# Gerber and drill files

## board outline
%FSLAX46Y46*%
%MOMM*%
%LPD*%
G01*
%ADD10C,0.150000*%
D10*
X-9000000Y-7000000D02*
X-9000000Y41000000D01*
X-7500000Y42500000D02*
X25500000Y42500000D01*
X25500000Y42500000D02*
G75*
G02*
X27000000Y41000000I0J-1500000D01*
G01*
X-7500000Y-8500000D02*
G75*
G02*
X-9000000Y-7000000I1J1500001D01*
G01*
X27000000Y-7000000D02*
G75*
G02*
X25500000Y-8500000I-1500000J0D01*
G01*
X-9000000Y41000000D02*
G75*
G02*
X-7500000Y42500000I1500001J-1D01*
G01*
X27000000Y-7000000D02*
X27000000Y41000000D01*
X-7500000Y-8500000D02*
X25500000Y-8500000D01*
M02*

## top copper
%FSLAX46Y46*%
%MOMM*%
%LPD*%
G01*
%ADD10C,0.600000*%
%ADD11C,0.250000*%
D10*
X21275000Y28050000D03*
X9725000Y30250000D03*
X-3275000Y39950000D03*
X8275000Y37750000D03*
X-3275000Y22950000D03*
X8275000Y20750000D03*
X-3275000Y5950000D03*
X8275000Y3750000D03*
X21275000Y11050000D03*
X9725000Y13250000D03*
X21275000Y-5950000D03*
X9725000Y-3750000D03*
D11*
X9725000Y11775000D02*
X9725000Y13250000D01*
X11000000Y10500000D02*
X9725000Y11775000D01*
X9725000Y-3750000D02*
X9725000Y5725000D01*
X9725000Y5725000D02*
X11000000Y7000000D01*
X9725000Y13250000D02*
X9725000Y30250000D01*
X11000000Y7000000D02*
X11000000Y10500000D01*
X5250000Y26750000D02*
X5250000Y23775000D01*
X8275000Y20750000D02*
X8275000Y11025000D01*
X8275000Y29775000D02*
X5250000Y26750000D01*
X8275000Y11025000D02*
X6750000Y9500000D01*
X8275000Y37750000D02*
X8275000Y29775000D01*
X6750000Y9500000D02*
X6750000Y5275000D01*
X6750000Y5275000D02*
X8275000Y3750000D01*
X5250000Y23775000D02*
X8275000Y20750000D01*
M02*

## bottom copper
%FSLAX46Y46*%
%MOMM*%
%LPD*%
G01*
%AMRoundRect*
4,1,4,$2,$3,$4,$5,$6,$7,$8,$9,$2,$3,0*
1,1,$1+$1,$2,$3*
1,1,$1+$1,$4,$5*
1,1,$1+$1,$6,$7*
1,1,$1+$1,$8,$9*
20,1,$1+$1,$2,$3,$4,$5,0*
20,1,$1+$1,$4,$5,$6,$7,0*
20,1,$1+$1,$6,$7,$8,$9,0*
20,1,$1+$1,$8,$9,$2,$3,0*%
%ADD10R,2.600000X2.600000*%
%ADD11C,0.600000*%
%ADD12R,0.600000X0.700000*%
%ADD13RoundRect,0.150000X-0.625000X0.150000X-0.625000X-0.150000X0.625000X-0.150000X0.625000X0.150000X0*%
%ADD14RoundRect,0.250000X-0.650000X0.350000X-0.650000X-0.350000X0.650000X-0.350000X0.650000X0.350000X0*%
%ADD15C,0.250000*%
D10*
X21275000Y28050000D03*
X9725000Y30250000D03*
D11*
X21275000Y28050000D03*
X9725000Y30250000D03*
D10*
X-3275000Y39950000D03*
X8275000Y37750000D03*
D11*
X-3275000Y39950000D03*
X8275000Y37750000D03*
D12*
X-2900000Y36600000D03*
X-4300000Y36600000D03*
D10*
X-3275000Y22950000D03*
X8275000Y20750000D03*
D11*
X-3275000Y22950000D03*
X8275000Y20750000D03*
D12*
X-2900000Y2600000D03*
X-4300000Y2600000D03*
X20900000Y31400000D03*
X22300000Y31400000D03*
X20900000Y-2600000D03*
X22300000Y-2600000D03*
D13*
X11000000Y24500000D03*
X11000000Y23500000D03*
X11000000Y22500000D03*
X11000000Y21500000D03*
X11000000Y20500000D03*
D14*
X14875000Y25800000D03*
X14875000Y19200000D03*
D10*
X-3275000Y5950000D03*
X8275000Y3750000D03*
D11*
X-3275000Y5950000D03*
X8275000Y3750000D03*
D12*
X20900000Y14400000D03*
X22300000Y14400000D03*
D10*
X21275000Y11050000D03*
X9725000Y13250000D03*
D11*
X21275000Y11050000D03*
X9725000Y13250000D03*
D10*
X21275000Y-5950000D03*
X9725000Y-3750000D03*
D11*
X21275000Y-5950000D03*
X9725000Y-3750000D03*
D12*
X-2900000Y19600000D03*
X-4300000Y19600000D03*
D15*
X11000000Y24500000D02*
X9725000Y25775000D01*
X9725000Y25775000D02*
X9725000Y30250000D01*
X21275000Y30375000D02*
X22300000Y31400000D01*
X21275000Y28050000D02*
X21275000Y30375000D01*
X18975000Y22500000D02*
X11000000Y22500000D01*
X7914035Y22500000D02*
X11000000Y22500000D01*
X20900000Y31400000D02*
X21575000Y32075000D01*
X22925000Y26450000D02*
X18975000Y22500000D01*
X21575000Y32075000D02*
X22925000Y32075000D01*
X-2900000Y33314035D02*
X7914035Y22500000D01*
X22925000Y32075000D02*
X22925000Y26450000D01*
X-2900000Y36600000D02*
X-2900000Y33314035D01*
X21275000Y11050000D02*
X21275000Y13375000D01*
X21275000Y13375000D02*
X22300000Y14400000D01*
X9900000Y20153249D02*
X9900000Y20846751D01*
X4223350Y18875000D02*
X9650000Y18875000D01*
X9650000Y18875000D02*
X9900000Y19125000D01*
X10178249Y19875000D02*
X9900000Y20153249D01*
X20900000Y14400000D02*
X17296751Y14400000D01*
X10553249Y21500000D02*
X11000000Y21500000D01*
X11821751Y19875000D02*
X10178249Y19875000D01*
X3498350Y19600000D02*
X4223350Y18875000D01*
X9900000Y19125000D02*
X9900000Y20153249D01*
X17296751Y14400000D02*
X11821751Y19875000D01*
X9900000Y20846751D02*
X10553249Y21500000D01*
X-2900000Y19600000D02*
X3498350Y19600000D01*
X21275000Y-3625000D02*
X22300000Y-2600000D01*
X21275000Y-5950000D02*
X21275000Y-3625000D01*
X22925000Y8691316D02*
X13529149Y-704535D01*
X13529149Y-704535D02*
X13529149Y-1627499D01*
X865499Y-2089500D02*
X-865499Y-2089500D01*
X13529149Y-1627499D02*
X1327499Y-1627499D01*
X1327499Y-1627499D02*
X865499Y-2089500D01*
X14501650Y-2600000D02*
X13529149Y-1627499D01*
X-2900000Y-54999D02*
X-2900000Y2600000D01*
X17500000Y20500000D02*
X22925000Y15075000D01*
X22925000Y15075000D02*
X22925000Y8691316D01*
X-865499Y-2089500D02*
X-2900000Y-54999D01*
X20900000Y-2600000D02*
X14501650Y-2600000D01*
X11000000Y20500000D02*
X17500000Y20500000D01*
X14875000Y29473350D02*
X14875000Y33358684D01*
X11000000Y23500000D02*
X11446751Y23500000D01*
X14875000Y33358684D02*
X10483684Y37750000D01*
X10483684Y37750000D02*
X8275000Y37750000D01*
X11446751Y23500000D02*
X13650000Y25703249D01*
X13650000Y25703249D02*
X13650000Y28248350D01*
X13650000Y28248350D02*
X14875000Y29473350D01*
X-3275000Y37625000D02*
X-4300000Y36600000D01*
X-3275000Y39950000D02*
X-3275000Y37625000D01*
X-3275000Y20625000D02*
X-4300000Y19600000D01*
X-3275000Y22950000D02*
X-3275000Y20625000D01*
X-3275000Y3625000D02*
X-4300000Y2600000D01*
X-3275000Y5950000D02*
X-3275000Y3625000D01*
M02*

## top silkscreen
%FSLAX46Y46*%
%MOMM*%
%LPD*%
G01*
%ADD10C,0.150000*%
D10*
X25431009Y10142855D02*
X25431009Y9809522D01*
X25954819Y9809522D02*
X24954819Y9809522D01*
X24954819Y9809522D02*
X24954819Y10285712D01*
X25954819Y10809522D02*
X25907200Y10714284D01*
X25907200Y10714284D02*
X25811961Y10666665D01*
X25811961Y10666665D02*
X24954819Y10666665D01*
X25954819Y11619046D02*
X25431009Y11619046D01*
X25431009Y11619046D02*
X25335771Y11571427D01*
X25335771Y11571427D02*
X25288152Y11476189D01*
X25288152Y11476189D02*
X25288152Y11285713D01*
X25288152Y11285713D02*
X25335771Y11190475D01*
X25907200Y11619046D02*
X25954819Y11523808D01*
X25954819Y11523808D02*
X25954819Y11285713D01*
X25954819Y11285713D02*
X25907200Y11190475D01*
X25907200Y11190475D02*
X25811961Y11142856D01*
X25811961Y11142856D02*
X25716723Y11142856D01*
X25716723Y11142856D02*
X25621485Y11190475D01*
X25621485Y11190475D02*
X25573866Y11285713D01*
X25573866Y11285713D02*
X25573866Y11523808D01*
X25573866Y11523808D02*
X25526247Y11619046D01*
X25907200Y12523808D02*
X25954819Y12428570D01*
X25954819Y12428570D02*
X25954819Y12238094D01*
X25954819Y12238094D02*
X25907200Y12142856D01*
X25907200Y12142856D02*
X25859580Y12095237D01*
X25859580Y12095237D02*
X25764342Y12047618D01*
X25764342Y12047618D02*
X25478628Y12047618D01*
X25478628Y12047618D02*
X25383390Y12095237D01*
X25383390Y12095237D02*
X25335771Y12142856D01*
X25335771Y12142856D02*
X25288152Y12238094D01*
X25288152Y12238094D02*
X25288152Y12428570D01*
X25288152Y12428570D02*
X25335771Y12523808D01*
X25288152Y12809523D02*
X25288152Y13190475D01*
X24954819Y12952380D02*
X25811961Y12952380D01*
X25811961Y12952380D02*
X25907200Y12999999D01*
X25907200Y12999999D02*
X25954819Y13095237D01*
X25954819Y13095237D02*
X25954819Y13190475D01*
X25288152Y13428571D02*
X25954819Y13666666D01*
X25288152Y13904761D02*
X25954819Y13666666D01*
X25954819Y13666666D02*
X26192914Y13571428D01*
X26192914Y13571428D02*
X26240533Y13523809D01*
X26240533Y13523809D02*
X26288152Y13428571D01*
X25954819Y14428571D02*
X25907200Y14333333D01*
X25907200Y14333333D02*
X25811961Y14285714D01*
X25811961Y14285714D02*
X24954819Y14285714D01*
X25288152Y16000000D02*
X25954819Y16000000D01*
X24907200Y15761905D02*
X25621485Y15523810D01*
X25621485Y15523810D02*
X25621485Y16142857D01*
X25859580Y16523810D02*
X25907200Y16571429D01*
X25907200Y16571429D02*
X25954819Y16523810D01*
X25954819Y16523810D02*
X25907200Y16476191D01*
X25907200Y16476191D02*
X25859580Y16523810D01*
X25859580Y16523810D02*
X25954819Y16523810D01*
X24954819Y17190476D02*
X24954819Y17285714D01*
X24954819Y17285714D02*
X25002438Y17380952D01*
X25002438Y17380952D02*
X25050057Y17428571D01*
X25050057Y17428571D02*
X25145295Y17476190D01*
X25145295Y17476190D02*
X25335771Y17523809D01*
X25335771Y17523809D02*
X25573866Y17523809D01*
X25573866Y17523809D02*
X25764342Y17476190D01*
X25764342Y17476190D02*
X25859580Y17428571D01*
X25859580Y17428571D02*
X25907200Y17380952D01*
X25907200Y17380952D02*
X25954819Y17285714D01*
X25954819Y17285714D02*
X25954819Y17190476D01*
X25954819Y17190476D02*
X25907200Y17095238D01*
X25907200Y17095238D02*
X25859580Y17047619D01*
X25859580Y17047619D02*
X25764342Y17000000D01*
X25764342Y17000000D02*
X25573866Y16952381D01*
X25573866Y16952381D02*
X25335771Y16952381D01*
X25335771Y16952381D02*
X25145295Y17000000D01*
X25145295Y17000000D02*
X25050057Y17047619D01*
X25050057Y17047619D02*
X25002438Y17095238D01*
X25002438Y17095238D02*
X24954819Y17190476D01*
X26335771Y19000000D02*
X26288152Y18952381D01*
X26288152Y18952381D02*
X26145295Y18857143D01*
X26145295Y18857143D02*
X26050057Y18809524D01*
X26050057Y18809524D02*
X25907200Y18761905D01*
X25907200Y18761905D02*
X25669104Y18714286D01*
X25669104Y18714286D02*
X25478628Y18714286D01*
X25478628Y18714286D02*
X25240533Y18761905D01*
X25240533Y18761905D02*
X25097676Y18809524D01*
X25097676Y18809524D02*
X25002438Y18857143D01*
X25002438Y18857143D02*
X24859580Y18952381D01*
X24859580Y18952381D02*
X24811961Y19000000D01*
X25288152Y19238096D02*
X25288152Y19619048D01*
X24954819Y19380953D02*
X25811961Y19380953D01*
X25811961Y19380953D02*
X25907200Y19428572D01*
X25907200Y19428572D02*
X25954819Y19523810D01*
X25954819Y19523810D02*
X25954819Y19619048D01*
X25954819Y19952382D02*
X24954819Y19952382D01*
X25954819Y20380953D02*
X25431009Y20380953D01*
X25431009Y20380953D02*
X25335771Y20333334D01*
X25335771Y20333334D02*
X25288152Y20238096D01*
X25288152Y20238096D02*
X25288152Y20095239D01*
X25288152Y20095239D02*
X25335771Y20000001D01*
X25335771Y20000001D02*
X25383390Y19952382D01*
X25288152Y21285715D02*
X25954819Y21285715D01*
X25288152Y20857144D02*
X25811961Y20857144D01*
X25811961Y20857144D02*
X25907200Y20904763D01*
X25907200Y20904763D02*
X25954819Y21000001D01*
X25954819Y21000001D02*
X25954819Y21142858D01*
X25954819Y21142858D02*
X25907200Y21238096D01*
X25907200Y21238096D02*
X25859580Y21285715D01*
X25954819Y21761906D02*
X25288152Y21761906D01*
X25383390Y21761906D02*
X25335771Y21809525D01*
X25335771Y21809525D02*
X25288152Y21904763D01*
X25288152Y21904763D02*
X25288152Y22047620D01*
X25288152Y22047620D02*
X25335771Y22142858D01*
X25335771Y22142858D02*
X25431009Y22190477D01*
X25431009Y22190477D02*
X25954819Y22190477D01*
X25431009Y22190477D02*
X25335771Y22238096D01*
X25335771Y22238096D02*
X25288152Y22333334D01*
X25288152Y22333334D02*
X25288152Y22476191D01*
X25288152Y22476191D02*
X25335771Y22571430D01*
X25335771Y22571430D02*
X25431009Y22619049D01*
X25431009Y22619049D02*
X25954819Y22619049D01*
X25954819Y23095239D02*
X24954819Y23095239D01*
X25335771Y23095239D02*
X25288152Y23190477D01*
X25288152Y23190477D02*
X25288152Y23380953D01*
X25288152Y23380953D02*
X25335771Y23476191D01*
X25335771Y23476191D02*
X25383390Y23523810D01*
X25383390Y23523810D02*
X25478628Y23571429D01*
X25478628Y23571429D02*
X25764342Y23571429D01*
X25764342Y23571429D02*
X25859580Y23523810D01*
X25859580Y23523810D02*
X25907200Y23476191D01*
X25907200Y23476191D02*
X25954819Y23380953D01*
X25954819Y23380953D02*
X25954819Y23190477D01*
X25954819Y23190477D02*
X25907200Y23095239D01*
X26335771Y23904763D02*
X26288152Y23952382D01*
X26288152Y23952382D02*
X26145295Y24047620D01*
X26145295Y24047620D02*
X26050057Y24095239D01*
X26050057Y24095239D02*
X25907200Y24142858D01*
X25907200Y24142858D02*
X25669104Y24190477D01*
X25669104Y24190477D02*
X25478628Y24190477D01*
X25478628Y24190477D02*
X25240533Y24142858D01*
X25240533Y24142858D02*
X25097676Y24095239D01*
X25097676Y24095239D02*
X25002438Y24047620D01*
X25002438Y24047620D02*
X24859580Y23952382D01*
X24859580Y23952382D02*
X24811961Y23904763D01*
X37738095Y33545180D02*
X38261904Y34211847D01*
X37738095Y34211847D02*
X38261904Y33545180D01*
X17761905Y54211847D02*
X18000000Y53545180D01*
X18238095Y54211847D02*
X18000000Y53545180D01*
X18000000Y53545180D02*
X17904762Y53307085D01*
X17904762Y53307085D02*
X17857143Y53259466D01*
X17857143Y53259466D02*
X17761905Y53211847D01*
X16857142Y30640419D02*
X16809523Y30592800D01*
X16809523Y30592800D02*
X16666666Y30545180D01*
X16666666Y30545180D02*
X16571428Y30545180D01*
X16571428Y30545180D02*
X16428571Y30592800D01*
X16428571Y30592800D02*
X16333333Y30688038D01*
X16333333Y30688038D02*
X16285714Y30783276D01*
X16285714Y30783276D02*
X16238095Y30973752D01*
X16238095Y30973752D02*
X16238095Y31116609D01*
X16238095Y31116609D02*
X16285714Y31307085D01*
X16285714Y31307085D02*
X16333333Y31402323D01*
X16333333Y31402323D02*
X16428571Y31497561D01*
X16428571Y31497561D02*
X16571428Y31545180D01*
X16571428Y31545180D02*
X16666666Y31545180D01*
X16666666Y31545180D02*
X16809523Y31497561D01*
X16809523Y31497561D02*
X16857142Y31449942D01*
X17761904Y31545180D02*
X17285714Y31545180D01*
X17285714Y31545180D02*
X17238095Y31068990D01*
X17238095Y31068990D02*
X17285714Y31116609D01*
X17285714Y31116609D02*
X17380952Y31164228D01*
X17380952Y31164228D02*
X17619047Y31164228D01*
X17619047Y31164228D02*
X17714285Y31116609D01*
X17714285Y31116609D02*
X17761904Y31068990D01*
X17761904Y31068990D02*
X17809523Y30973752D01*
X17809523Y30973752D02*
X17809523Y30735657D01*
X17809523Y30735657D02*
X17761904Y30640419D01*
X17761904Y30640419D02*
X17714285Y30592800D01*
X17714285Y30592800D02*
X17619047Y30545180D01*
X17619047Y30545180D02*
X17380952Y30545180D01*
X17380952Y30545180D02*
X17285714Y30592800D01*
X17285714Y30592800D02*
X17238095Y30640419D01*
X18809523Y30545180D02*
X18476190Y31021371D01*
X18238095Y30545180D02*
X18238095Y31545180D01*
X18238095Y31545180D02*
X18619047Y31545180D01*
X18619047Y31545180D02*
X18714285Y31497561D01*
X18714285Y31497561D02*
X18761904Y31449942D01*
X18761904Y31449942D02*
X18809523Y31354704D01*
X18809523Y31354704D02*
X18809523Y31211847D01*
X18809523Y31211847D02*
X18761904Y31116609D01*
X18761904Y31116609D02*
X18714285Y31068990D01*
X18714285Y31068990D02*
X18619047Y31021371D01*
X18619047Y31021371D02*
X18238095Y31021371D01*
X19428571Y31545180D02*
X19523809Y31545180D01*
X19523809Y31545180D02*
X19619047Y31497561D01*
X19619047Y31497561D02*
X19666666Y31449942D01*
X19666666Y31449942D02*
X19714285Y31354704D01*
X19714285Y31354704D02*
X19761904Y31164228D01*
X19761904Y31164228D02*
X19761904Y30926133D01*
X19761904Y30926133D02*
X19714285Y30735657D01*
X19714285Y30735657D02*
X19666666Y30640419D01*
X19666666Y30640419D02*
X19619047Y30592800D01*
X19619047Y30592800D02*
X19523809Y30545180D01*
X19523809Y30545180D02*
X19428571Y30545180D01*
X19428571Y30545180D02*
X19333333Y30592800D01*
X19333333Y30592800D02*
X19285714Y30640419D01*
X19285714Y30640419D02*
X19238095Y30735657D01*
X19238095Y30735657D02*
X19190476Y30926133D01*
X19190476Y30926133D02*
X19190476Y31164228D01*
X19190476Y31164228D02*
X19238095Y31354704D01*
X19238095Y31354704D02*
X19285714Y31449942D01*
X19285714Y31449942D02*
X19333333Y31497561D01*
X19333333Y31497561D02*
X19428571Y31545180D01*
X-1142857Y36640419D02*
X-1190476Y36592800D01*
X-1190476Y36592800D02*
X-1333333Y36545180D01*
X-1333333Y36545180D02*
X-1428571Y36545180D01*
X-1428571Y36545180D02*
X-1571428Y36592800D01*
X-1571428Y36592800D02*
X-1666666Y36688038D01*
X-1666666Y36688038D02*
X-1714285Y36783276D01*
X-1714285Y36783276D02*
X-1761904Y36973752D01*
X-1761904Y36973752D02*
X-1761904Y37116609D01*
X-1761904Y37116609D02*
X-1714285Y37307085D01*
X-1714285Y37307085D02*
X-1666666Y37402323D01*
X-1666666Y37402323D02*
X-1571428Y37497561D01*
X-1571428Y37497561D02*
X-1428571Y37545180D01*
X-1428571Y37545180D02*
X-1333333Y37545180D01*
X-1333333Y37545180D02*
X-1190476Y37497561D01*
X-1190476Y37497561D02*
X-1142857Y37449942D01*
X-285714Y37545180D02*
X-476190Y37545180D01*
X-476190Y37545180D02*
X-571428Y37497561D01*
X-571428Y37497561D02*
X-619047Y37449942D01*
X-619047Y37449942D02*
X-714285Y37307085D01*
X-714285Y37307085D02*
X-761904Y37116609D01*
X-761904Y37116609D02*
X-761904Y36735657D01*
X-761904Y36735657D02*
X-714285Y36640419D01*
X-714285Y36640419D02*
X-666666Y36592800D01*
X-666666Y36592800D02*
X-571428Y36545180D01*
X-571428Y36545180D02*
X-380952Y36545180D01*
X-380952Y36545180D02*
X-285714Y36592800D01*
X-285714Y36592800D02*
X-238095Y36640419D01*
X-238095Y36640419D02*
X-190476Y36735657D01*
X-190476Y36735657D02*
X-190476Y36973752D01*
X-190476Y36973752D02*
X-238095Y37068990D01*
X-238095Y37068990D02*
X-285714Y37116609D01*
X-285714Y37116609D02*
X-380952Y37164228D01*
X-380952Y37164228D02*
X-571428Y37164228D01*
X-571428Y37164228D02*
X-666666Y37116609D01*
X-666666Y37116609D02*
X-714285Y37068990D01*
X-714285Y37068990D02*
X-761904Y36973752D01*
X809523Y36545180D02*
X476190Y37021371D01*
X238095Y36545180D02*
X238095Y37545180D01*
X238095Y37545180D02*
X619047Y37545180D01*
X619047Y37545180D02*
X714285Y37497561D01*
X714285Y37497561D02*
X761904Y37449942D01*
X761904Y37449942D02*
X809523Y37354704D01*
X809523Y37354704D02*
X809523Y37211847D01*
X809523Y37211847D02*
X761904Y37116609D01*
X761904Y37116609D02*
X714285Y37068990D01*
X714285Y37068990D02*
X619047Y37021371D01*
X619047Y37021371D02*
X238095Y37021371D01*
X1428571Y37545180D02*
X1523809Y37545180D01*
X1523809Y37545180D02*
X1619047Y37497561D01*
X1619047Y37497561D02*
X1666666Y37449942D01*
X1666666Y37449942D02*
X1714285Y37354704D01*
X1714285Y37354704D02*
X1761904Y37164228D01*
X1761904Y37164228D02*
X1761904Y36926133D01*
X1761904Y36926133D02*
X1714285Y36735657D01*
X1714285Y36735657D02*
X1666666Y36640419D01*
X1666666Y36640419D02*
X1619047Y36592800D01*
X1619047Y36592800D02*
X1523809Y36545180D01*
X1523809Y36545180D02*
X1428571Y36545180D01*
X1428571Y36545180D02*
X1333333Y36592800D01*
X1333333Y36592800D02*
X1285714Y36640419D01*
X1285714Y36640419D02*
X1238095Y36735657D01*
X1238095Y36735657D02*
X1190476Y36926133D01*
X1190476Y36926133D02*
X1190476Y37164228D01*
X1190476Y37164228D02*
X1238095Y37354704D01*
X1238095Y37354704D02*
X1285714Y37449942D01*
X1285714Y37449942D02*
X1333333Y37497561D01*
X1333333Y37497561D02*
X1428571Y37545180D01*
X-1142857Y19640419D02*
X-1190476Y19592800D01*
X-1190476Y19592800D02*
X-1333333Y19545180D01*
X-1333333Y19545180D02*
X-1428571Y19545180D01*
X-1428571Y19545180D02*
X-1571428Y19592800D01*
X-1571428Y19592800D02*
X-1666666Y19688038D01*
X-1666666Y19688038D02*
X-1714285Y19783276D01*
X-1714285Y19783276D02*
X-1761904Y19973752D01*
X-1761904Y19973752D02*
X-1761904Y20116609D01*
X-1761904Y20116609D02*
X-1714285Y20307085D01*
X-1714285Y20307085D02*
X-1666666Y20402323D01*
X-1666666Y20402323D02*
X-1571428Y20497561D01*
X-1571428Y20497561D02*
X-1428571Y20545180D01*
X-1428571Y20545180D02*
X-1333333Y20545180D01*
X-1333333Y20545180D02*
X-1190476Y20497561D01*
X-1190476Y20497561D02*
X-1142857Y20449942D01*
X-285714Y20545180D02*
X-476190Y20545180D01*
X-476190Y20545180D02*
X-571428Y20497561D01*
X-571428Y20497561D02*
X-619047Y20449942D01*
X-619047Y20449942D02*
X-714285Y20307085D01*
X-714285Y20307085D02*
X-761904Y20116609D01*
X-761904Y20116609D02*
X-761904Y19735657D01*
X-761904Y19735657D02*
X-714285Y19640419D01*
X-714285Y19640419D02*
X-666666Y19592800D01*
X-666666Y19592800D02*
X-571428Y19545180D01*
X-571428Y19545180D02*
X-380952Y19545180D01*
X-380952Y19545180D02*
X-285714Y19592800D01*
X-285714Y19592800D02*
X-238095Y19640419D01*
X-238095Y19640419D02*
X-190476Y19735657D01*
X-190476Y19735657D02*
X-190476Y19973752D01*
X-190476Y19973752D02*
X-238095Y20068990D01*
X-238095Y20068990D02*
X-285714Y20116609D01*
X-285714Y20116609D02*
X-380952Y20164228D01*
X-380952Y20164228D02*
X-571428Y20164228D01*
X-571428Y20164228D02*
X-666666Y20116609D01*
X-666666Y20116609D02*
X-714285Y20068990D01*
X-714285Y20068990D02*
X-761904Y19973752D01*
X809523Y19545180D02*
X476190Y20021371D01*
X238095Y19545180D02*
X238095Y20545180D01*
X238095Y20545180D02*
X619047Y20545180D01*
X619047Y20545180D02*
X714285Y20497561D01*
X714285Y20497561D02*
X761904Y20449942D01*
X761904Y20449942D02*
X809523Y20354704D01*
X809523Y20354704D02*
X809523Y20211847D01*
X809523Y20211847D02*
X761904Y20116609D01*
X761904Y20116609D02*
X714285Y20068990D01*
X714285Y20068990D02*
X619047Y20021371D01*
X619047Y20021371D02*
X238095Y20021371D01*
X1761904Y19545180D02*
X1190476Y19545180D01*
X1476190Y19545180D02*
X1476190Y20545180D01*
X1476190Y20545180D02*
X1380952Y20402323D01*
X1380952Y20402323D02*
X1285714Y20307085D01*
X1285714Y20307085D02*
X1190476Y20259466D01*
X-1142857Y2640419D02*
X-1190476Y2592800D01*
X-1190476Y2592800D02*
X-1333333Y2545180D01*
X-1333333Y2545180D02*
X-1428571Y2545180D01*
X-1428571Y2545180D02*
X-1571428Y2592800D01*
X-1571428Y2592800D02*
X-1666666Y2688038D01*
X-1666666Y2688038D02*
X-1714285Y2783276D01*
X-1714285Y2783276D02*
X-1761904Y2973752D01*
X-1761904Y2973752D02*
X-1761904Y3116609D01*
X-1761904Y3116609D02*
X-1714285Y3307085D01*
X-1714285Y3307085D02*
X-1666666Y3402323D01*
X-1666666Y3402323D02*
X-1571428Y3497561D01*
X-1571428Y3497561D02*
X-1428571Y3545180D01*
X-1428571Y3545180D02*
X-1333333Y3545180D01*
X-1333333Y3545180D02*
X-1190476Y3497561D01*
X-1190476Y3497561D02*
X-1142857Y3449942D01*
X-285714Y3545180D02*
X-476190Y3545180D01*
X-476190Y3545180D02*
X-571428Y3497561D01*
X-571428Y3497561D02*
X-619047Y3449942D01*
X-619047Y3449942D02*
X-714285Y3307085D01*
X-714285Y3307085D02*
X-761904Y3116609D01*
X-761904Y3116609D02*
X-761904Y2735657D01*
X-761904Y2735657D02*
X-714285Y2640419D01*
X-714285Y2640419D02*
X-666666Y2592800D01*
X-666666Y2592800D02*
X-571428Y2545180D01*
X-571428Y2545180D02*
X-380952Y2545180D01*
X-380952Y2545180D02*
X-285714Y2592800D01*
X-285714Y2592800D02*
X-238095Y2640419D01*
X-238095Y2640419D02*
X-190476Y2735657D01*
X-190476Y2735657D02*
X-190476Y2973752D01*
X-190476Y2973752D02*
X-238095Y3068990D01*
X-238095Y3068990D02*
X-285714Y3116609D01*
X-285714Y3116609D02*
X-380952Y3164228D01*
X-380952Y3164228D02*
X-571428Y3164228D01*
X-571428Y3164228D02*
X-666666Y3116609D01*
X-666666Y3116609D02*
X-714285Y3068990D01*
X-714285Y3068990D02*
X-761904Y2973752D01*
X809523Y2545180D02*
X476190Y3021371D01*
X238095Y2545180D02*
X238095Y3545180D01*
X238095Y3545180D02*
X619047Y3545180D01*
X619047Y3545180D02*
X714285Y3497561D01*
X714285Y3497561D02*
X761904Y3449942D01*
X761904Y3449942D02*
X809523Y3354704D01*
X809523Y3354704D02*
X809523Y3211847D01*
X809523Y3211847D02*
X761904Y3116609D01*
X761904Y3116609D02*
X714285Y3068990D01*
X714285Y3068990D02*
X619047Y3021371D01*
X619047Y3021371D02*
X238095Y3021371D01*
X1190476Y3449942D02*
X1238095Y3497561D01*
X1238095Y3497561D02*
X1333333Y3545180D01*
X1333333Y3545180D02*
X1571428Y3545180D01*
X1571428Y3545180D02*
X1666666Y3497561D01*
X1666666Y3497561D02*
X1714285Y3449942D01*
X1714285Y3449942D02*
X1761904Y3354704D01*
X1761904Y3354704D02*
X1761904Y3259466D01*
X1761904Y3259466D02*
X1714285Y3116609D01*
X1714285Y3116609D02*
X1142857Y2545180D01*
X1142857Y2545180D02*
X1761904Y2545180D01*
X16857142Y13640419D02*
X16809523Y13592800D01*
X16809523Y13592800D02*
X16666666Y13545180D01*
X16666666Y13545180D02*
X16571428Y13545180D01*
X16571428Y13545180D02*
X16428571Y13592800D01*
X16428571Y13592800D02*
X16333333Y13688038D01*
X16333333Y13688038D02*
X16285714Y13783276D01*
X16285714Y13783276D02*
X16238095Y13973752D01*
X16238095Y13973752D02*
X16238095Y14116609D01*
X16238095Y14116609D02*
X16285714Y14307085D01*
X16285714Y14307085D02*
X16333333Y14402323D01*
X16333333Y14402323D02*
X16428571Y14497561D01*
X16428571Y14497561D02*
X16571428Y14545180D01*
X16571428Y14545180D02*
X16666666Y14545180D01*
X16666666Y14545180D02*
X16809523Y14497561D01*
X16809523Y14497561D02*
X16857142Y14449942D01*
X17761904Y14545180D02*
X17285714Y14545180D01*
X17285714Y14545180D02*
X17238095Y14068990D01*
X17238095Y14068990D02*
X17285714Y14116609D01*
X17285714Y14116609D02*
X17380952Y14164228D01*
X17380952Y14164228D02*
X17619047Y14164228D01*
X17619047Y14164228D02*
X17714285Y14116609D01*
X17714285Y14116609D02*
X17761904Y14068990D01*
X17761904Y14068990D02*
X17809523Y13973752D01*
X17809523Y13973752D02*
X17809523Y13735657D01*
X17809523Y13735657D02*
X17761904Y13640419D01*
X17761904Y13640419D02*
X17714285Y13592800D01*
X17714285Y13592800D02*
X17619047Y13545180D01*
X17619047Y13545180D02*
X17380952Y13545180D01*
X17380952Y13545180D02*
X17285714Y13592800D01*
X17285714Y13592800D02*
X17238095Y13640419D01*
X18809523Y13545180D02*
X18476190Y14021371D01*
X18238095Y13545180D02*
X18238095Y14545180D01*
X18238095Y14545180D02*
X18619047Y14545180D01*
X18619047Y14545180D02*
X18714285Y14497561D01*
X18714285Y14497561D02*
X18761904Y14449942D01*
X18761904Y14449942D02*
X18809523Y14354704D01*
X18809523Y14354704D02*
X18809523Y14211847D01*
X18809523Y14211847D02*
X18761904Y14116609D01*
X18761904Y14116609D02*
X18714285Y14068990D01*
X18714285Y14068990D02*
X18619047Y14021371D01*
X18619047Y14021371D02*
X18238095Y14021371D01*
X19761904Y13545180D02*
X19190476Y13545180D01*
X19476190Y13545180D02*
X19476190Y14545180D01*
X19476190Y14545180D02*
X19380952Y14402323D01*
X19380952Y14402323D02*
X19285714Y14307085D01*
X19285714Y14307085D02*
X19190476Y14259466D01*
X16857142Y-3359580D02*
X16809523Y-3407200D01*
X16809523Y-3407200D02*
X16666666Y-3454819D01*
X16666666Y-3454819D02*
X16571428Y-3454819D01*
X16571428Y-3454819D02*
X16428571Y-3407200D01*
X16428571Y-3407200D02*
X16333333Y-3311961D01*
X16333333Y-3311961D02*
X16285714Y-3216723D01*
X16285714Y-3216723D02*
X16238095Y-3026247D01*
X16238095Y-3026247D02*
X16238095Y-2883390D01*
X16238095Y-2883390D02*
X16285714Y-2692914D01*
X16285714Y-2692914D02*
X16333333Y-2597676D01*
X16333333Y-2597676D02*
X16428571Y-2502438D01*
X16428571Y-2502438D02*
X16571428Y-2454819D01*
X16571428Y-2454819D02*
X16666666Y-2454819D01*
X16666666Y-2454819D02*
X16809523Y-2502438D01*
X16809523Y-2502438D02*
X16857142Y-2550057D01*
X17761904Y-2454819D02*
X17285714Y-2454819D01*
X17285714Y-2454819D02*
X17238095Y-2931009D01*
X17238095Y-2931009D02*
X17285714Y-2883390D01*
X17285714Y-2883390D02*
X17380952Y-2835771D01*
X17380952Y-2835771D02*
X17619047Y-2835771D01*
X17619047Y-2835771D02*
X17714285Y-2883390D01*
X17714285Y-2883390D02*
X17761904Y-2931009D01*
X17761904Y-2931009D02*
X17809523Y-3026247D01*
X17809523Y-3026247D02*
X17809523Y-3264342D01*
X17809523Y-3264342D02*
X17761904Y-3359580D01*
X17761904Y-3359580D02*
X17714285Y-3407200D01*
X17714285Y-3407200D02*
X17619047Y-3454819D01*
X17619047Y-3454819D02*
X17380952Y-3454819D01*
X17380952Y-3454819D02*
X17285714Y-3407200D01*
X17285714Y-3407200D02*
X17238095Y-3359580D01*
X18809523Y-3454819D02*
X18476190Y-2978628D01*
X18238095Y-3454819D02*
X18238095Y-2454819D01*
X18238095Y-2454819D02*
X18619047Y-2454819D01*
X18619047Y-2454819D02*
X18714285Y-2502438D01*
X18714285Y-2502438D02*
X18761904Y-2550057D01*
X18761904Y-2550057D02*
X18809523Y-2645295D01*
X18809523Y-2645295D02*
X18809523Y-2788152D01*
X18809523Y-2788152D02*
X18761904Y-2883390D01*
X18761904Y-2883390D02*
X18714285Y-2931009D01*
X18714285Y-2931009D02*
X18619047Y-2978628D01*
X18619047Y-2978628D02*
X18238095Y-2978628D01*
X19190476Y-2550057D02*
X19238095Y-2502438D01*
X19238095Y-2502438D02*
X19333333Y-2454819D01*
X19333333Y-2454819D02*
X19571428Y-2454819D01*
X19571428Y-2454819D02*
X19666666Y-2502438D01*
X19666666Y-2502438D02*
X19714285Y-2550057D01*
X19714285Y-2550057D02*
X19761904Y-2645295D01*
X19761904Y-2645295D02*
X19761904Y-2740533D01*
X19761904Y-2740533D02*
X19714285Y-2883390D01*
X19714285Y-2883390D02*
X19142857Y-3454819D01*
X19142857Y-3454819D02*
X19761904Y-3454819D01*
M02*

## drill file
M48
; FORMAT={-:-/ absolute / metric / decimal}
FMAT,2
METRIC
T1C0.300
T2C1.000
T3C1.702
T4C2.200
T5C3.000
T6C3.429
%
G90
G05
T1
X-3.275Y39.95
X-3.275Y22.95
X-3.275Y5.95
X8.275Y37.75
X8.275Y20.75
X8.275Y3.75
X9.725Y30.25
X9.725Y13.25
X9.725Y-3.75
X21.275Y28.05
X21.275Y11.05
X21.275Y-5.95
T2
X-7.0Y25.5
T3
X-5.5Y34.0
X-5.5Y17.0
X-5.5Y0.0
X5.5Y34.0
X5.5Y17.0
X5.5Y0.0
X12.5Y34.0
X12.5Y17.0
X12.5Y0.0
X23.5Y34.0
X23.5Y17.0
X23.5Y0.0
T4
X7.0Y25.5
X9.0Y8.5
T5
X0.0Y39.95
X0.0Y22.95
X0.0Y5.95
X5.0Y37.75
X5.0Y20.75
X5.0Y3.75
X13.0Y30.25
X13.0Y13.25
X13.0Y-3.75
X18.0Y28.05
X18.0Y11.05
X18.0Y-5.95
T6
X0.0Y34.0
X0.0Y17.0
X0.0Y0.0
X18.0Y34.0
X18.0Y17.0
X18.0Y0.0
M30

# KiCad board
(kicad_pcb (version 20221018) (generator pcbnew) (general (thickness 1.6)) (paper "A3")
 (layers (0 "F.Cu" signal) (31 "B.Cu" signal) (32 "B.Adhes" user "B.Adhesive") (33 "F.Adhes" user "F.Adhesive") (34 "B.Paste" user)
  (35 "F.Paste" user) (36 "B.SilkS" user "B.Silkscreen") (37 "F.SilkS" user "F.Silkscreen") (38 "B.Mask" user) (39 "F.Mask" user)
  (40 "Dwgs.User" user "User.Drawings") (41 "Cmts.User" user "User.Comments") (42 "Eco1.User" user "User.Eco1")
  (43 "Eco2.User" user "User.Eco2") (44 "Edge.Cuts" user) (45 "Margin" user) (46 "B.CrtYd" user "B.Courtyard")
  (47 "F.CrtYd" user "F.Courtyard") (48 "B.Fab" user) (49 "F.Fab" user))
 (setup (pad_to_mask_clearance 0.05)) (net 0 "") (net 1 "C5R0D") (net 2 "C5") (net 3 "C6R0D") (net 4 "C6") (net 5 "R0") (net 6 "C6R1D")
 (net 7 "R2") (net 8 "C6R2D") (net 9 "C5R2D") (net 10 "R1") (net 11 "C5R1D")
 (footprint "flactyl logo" (layer "F.Cu") (at 25.5 -17 -90)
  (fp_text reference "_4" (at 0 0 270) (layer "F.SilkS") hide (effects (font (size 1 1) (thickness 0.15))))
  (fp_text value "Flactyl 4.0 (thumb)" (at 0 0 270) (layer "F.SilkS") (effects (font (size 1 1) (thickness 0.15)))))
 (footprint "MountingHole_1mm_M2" (layer "F.Cu") (at -7 -25.5)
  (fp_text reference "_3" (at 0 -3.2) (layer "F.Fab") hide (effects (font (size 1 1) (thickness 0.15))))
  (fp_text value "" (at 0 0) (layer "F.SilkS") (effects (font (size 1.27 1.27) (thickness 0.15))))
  (pad "" np_thru_hole circle (at 0 0) (size 1 1) (drill 1) (layers "*.Cu" "*.Mask")))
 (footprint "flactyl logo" (layer "F.Cu") (at 38 -34)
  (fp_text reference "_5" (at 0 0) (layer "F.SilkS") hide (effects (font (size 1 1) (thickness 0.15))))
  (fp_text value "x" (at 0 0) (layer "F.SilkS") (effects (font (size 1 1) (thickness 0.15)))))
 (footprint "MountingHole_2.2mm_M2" (layer "F.Cu") (at 7 -25.5)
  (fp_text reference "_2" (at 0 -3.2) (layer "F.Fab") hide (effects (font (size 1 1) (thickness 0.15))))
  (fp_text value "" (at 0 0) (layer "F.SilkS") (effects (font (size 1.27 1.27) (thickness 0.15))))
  (pad "" np_thru_hole circle (at 0 0) (size 2.2 2.2) (drill 2.2) (layers "*.Cu" "*.Mask")))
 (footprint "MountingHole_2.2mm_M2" (layer "F.Cu") (at 9 -8.5)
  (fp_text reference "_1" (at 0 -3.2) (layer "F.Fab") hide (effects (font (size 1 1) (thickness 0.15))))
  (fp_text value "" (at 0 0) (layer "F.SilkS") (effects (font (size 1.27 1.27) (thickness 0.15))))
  (pad "" np_thru_hole circle (at 0 0) (size 2.2 2.2) (drill 2.2) (layers "*.Cu" "*.Mask")))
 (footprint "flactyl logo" (layer "F.Cu") (at 18 -54)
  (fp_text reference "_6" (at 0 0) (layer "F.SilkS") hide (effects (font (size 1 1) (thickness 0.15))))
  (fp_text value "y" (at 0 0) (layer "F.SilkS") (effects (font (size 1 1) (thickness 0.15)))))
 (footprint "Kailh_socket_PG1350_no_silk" (layer "B.Cu") (at 18 -34)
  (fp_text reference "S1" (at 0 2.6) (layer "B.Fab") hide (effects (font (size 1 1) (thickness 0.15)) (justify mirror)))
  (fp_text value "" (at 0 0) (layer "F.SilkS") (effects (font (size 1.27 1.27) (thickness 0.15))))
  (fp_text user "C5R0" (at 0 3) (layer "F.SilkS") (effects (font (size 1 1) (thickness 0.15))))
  (pad "" np_thru_hole circle (at -5.5 0) (size 1.7018 1.7018) (drill 1.7018) (layers "*.Cu" "*.Mask"))
  (pad "" np_thru_hole circle (at -5 3.75) (size 3 3) (drill 3) (layers "*.Cu" "*.Mask"))
  (pad "" np_thru_hole circle (at 0 0) (size 3.429 3.429) (drill 3.429) (layers "*.Cu" "*.Mask"))
  (pad "" np_thru_hole circle (at 0 5.95) (size 3 3) (drill 3) (layers "*.Cu" "*.Mask"))
  (pad "" np_thru_hole circle (at 5.5 0) (size 1.7018 1.7018) (drill 1.7018) (layers "*.Cu" "*.Mask"))
  (pad "1" smd rect (at 3.275 5.95) (size 2.6 2.6) (layers "B.Cu" "B.Paste" "B.Mask") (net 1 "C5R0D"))
  (pad "2" smd rect (at -8.275 3.75) (size 2.6 2.6) (layers "B.Cu" "B.Paste" "B.Mask") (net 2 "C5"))
  (pad "3" thru_hole circle (at 3.275 5.95) (size 0.6 0.6) (drill 0.3) (layers "*.Cu") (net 1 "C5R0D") (zone_connect 2))
  (pad "4" thru_hole circle (at -8.275 3.75) (size 0.6 0.6) (drill 0.3) (layers "*.Cu") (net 2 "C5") (zone_connect 2)))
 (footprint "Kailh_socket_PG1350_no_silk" (layer "B.Cu") (at 0 -34 180)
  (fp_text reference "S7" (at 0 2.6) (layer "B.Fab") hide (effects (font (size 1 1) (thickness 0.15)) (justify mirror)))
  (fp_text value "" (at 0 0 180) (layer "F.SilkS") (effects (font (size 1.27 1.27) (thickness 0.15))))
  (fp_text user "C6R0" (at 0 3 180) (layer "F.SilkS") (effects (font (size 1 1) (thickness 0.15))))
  (pad "" np_thru_hole circle (at -5.5 0) (size 1.7018 1.7018) (drill 1.7018) (layers "*.Cu" "*.Mask"))
  (pad "" np_thru_hole circle (at -5 3.75) (size 3 3) (drill 3) (layers "*.Cu" "*.Mask"))
  (pad "" np_thru_hole circle (at 0 0) (size 3.429 3.429) (drill 3.429) (layers "*.Cu" "*.Mask"))
  (pad "" np_thru_hole circle (at 0 5.95) (size 3 3) (drill 3) (layers "*.Cu" "*.Mask"))
  (pad "" np_thru_hole circle (at 5.5 0) (size 1.7018 1.7018) (drill 1.7018) (layers "*.Cu" "*.Mask"))
  (pad "1" smd rect (at 3.275 5.95) (size 2.6 2.6) (layers "B.Cu" "B.Paste" "B.Mask") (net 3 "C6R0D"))
  (pad "2" smd rect (at -8.275 3.75) (size 2.6 2.6) (layers "B.Cu" "B.Paste" "B.Mask") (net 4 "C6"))
  (pad "3" thru_hole circle (at 3.275 5.95) (size 0.6 0.6) (drill 0.3) (layers "*.Cu") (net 3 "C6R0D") (zone_connect 2))
  (pad "4" thru_hole circle (at -8.275 3.75) (size 0.6 0.6) (drill 0.3) (layers "*.Cu") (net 4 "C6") (zone_connect 2)))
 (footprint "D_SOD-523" (layer "B.Cu") (at -3.6 -36.6 180)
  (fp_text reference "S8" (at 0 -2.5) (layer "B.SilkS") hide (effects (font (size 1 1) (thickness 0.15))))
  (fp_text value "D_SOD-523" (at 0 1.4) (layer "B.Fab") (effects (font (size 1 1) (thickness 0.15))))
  (pad "1" smd rect (at -0.7 0 180) (size 0.6 0.7) (layers "B.Cu" "B.Paste" "B.Mask") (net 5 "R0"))
  (pad "2" smd rect (at 0.7 0 180) (size 0.6 0.7) (layers "B.Cu" "B.Paste" "B.Mask") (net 3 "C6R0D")))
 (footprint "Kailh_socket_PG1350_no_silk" (layer "B.Cu") (at 0 -17 180)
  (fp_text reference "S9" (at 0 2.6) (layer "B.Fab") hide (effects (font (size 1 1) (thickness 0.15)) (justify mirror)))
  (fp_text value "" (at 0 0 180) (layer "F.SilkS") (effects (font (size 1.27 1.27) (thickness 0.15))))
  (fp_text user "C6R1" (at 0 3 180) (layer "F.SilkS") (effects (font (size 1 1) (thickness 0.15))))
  (pad "" np_thru_hole circle (at -5.5 0) (size 1.7018 1.7018) (drill 1.7018) (layers "*.Cu" "*.Mask"))
  (pad "" np_thru_hole circle (at -5 3.75) (size 3 3) (drill 3) (layers "*.Cu" "*.Mask"))
  (pad "" np_thru_hole circle (at 0 0) (size 3.429 3.429) (drill 3.429) (layers "*.Cu" "*.Mask"))
  (pad "" np_thru_hole circle (at 0 5.95) (size 3 3) (drill 3) (layers "*.Cu" "*.Mask"))
  (pad "" np_thru_hole circle (at 5.5 0) (size 1.7018 1.7018) (drill 1.7018) (layers "*.Cu" "*.Mask"))
  (pad "1" smd rect (at 3.275 5.95) (size 2.6 2.6) (layers "B.Cu" "B.Paste" "B.Mask") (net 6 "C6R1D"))
  (pad "2" smd rect (at -8.275 3.75) (size 2.6 2.6) (layers "B.Cu" "B.Paste" "B.Mask") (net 4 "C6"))
  (pad "3" thru_hole circle (at 3.275 5.95) (size 0.6 0.6) (drill 0.3) (layers "*.Cu") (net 6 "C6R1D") (zone_connect 2))
  (pad "4" thru_hole circle (at -8.275 3.75) (size 0.6 0.6) (drill 0.3) (layers "*.Cu") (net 4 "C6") (zone_connect 2)))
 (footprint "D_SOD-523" (layer "B.Cu") (at -3.6 -2.6 180)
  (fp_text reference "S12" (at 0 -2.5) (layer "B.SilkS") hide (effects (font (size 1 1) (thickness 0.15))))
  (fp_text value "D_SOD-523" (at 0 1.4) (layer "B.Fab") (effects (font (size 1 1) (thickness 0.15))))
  (pad "1" smd rect (at -0.7 0 180) (size 0.6 0.7) (layers "B.Cu" "B.Paste" "B.Mask") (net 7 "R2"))
  (pad "2" smd rect (at 0.7 0 180) (size 0.6 0.7) (layers "B.Cu" "B.Paste" "B.Mask") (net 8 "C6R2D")))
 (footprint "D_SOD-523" (layer "B.Cu") (at 21.6 -31.4)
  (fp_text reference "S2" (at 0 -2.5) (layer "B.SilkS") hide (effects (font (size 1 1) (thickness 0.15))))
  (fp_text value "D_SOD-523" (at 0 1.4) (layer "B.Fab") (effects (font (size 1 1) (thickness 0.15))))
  (pad "1" smd rect (at -0.7 0) (size 0.6 0.7) (layers "B.Cu" "B.Paste" "B.Mask") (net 5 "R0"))
  (pad "2" smd rect (at 0.7 0) (size 0.6 0.7) (layers "B.Cu" "B.Paste" "B.Mask") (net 1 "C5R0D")))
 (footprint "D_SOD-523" (layer "B.Cu") (at 21.6 2.6)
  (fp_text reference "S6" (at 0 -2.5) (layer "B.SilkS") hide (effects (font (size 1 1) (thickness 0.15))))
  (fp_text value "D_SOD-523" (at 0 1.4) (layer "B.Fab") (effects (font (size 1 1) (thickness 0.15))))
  (pad "1" smd rect (at -0.7 0) (size 0.6 0.7) (layers "B.Cu" "B.Paste" "B.Mask") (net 7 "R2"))
  (pad "2" smd rect (at 0.7 0) (size 0.6 0.7) (layers "B.Cu" "B.Paste" "B.Mask") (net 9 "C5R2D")))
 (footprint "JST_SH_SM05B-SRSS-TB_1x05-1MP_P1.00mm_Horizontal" (layer "B.Cu") (at 13 -22.5 -90)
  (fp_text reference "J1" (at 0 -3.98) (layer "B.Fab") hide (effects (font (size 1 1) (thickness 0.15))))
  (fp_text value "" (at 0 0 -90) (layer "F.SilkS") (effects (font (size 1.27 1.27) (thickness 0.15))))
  (pad "1" smd roundrect (at -2 2 270) (size 0.6 1.55) (layers "B.Cu" "B.Paste" "B.Mask") (roundrect_rratio 0.25) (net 2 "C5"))
  (pad "2" smd roundrect (at -1 2 270) (size 0.6 1.55) (layers "B.Cu" "B.Paste" "B.Mask") (roundrect_rratio 0.25) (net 4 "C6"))
  (pad "3" smd roundrect (at 0 2 270) (size 0.6 1.55) (layers "B.Cu" "B.Paste" "B.Mask") (roundrect_rratio 0.25) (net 5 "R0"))
  (pad "4" smd roundrect (at 1 2 270) (size 0.6 1.55) (layers "B.Cu" "B.Paste" "B.Mask") (roundrect_rratio 0.25) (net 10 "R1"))
  (pad "5" smd roundrect (at 2 2 270) (size 0.6 1.55) (layers "B.Cu" "B.Paste" "B.Mask") (roundrect_rratio 0.25) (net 7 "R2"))
  (pad "MP" smd roundrect (at -3.3 -1.875 270) (size 1.2 1.8) (layers "B.Cu" "B.Paste" "B.Mask") (roundrect_rratio 0.208333))
  (pad "MP" smd roundrect (at 3.3 -1.875 270) (size 1.2 1.8) (layers "B.Cu" "B.Paste" "B.Mask") (roundrect_rratio 0.208333)))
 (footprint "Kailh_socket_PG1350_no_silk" (layer "B.Cu") (at 0 0 180)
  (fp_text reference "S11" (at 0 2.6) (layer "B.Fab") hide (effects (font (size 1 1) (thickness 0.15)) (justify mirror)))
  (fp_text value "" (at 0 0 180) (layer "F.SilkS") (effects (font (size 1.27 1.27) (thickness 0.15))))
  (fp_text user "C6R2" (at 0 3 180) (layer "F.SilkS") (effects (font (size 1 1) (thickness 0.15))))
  (pad "" np_thru_hole circle (at -5.5 0) (size 1.7018 1.7018) (drill 1.7018) (layers "*.Cu" "*.Mask"))
  (pad "" np_thru_hole circle (at -5 3.75) (size 3 3) (drill 3) (layers "*.Cu" "*.Mask"))
  (pad "" np_thru_hole circle (at 0 0) (size 3.429 3.429) (drill 3.429) (layers "*.Cu" "*.Mask"))
  (pad "" np_thru_hole circle (at 0 5.95) (size 3 3) (drill 3) (layers "*.Cu" "*.Mask"))
  (pad "" np_thru_hole circle (at 5.5 0) (size 1.7018 1.7018) (drill 1.7018) (layers "*.Cu" "*.Mask"))
  (pad "1" smd rect (at 3.275 5.95) (size 2.6 2.6) (layers "B.Cu" "B.Paste" "B.Mask") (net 8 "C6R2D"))
  (pad "2" smd rect (at -8.275 3.75) (size 2.6 2.6) (layers "B.Cu" "B.Paste" "B.Mask") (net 4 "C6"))
  (pad "3" thru_hole circle (at 3.275 5.95) (size 0.6 0.6) (drill 0.3) (layers "*.Cu") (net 8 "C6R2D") (zone_connect 2))
  (pad "4" thru_hole circle (at -8.275 3.75) (size 0.6 0.6) (drill 0.3) (layers "*.Cu") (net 4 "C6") (zone_connect 2)))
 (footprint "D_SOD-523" (layer "B.Cu") (at 21.6 -14.4)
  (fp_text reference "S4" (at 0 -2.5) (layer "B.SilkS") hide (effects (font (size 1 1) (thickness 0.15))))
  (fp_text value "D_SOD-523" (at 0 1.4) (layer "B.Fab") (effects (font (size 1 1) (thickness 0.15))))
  (pad "1" smd rect (at -0.7 0) (size 0.6 0.7) (layers "B.Cu" "B.Paste" "B.Mask") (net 10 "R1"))
  (pad "2" smd rect (at 0.7 0) (size 0.6 0.7) (layers "B.Cu" "B.Paste" "B.Mask") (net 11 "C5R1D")))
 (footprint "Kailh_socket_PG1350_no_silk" (layer "B.Cu") (at 18 -17)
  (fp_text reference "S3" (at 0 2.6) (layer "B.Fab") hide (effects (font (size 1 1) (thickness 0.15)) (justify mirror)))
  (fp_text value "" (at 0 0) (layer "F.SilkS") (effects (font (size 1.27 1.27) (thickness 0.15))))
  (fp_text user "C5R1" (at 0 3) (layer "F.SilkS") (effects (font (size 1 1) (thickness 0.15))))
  (pad "" np_thru_hole circle (at -5.5 0) (size 1.7018 1.7018) (drill 1.7018) (layers "*.Cu" "*.Mask"))
  (pad "" np_thru_hole circle (at -5 3.75) (size 3 3) (drill 3) (layers "*.Cu" "*.Mask"))
  (pad "" np_thru_hole circle (at 0 0) (size 3.429 3.429) (drill 3.429) (layers "*.Cu" "*.Mask"))
  (pad "" np_thru_hole circle (at 0 5.95) (size 3 3) (drill 3) (layers "*.Cu" "*.Mask"))
  (pad "" np_thru_hole circle (at 5.5 0) (size 1.7018 1.7018) (drill 1.7018) (layers "*.Cu" "*.Mask"))
  (pad "1" smd rect (at 3.275 5.95) (size 2.6 2.6) (layers "B.Cu" "B.Paste" "B.Mask") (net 11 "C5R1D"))
  (pad "2" smd rect (at -8.275 3.75) (size 2.6 2.6) (layers "B.Cu" "B.Paste" "B.Mask") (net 2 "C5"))
  (pad "3" thru_hole circle (at 3.275 5.95) (size 0.6 0.6) (drill 0.3) (layers "*.Cu") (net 11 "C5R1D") (zone_connect 2))
  (pad "4" thru_hole circle (at -8.275 3.75) (size 0.6 0.6) (drill 0.3) (layers "*.Cu") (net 2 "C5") (zone_connect 2)))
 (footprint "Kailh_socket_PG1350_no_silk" (layer "B.Cu") (at 18 0)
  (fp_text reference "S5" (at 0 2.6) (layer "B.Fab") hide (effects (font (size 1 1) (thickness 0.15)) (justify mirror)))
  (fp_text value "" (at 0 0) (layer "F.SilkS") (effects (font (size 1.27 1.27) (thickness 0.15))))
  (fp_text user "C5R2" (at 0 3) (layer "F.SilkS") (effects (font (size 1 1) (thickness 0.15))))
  (pad "" np_thru_hole circle (at -5.5 0) (size 1.7018 1.7018) (drill 1.7018) (layers "*.Cu" "*.Mask"))
  (pad "" np_thru_hole circle (at -5 3.75) (size 3 3) (drill 3) (layers "*.Cu" "*.Mask"))
  (pad "" np_thru_hole circle (at 0 0) (size 3.429 3.429) (drill 3.429) (layers "*.Cu" "*.Mask"))
  (pad "" np_thru_hole circle (at 0 5.95) (size 3 3) (drill 3) (layers "*.Cu" "*.Mask"))
  (pad "" np_thru_hole circle (at 5.5 0) (size 1.7018 1.7018) (drill 1.7018) (layers "*.Cu" "*.Mask"))
  (pad "1" smd rect (at 3.275 5.95) (size 2.6 2.6) (layers "B.Cu" "B.Paste" "B.Mask") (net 9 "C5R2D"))
  (pad "2" smd rect (at -8.275 3.75) (size 2.6 2.6) (layers "B.Cu" "B.Paste" "B.Mask") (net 2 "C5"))
  (pad "3" thru_hole circle (at 3.275 5.95) (size 0.6 0.6) (drill 0.3) (layers "*.Cu") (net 9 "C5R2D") (zone_connect 2))
  (pad "4" thru_hole circle (at -8.275 3.75) (size 0.6 0.6) (drill 0.3) (layers "*.Cu") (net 2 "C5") (zone_connect 2)))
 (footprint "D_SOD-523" (layer "B.Cu") (at -3.6 -19.6 180)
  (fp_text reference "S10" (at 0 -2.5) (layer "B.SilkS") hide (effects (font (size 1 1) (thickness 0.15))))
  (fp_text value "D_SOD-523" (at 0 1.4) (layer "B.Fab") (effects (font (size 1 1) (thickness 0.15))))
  (pad "1" smd rect (at -0.7 0 180) (size 0.6 0.7) (layers "B.Cu" "B.Paste" "B.Mask") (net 10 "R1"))
  (pad "2" smd rect (at 0.7 0 180) (size 0.6 0.7) (layers "B.Cu" "B.Paste" "B.Mask") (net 6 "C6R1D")))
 (gr_line (start -9 7) (end -9 -41) (stroke (width 0.15) (type solid)) (layer "Edge.Cuts"))
 (gr_line (start -7.5 -42.5) (end 25.5 -42.5) (stroke (width 0.15) (type solid)) (layer "Edge.Cuts"))
 (gr_arc (start 25.5 -42.5) (mid 26.56066 -42.06066) (end 27 -41) (stroke (width 0.15) (type solid)) (layer "Edge.Cuts"))
 (gr_arc (start -7.5 8.5) (mid -8.56066 8.06066) (end -9 7) (stroke (width 0.15) (type solid)) (layer "Edge.Cuts"))
 (gr_arc (start 27 7) (mid 26.56066 8.06066) (end 25.5 8.5) (stroke (width 0.15) (type solid)) (layer "Edge.Cuts"))
 (gr_arc (start -9 -41) (mid -8.56066 -42.06066) (end -7.5 -42.5) (stroke (width 0.15) (type solid)) (layer "Edge.Cuts"))
 (gr_line (start 27 7) (end 27 -41) (stroke (width 0.15) (type solid)) (layer "Edge.Cuts"))
 (gr_line (start -7.5 8.5) (end 25.5 8.5) (stroke (width 0.15) (type solid)) (layer "Edge.Cuts"))
 (segment (start 9.725 -11.775) (end 9.725 -13.25) (width 0.25) (layer "F.Cu") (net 2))
 (segment (start 11 -10.5) (end 9.725 -11.775) (width 0.25) (layer "F.Cu") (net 2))
 (segment (start 9.725 3.75) (end 9.725 -5.725) (width 0.25) (layer "F.Cu") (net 2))
 (segment (start 9.725 -5.725) (end 11 -7) (width 0.25) (layer "F.Cu") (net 2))
 (segment (start 9.725 -13.25) (end 9.725 -30.25) (width 0.25) (layer "F.Cu") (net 2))
 (segment (start 11 -7) (end 11 -10.5) (width 0.25) (layer "F.Cu") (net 2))
 (segment (start 11 -24.5) (end 9.725 -25.775) (width 0.25) (layer "B.Cu") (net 2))
 (segment (start 9.725 -25.775) (end 9.725 -30.25) (width 0.25) (layer "B.Cu") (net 2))
 (segment (start 21.275 -30.375) (end 22.3 -31.4) (width 0.25) (layer "B.Cu") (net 1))
 (segment (start 21.275 -28.05) (end 21.275 -30.375) (width 0.25) (layer "B.Cu") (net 1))
 (segment (start 18.975 -22.5) (end 11 -22.5) (width 0.25) (layer "B.Cu") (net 5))
 (segment (start 7.914035 -22.5) (end 11 -22.5) (width 0.25) (layer "B.Cu") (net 5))
 (segment (start 20.9 -31.4) (end 21.575 -32.075) (width 0.25) (layer "B.Cu") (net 5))
 (segment (start 22.925 -26.45) (end 18.975 -22.5) (width 0.25) (layer "B.Cu") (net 5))
 (segment (start 21.575 -32.075) (end 22.925 -32.075) (width 0.25) (layer "B.Cu") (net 5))
 (segment (start -2.9 -33.314035) (end 7.914035 -22.5) (width 0.25) (layer "B.Cu") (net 5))
 (segment (start 22.925 -32.075) (end 22.925 -26.45) (width 0.25) (layer "B.Cu") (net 5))
 (segment (start -2.9 -36.6) (end -2.9 -33.314035) (width 0.25) (layer "B.Cu") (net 5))
 (segment (start 21.275 -11.05) (end 21.275 -13.375) (width 0.25) (layer "B.Cu") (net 11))
 (segment (start 21.275 -13.375) (end 22.3 -14.4) (width 0.25) (layer "B.Cu") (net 11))
 (segment (start 9.9 -20.153249) (end 9.9 -20.846751) (width 0.25) (layer "B.Cu") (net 10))
 (segment (start 4.22335 -18.875) (end 9.65 -18.875) (width 0.25) (layer "B.Cu") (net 10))
 (segment (start 9.65 -18.875) (end 9.9 -19.125) (width 0.25) (layer "B.Cu") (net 10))
 (segment (start 10.178249 -19.875) (end 9.9 -20.153249) (width 0.25) (layer "B.Cu") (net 10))
 (segment (start 20.9 -14.4) (end 17.296751 -14.4) (width 0.25) (layer "B.Cu") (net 10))
 (segment (start 10.553249 -21.5) (end 11 -21.5) (width 0.25) (layer "B.Cu") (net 10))
 (segment (start 11.821751 -19.875) (end 10.178249 -19.875) (width 0.25) (layer "B.Cu") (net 10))
 (segment (start 3.49835 -19.6) (end 4.22335 -18.875) (width 0.25) (layer "B.Cu") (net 10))
 (segment (start 9.9 -19.125) (end 9.9 -20.153249) (width 0.25) (layer "B.Cu") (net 10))
 (segment (start 17.296751 -14.4) (end 11.821751 -19.875) (width 0.25) (layer "B.Cu") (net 10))
 (segment (start 9.9 -20.846751) (end 10.553249 -21.5) (width 0.25) (layer "B.Cu") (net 10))
 (segment (start -2.9 -19.6) (end 3.49835 -19.6) (width 0.25) (layer "B.Cu") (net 10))
 (segment (start 21.275 3.625) (end 22.3 2.6) (width 0.25) (layer "B.Cu") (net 9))
 (segment (start 21.275 5.95) (end 21.275 3.625) (width 0.25) (layer "B.Cu") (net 9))
 (segment (start 22.925 -8.691316) (end 13.529149 0.704535) (width 0.25) (layer "B.Cu") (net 7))
 (segment (start 13.529149 0.704535) (end 13.529149 1.627499) (width 0.25) (layer "B.Cu") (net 7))
 (segment (start 0.865499 2.0895) (end -0.865499 2.0895) (width 0.25) (layer "B.Cu") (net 7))
 (segment (start 13.529149 1.627499) (end 1.327499 1.627499) (width 0.25) (layer "B.Cu") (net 7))
 (segment (start 1.327499 1.627499) (end 0.865499 2.0895) (width 0.25) (layer "B.Cu") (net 7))
 (segment (start 14.50165 2.6) (end 13.529149 1.627499) (width 0.25) (layer "B.Cu") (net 7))
 (segment (start -2.9 0.054999) (end -2.9 -2.6) (width 0.25) (layer "B.Cu") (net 7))
 (segment (start 17.5 -20.5) (end 22.925 -15.075) (width 0.25) (layer "B.Cu") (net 7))
 (segment (start 22.925 -15.075) (end 22.925 -8.691316) (width 0.25) (layer "B.Cu") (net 7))
 (segment (start -0.865499 2.0895) (end -2.9 0.054999) (width 0.25) (layer "B.Cu") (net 7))
 (segment (start 20.9 2.6) (end 14.50165 2.6) (width 0.25) (layer "B.Cu") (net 7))
 (segment (start 11 -20.5) (end 17.5 -20.5) (width 0.25) (layer "B.Cu") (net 7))
 (segment (start 5.25 -26.75) (end 5.25 -23.775) (width 0.25) (layer "F.Cu") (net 4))
 (segment (start 8.275 -20.75) (end 8.275 -11.025) (width 0.25) (layer "F.Cu") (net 4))
 (segment (start 8.275 -29.775) (end 5.25 -26.75) (width 0.25) (layer "F.Cu") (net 4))
 (segment (start 8.275 -11.025) (end 6.75 -9.5) (width 0.25) (layer "F.Cu") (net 4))
 (segment (start 8.275 -37.75) (end 8.275 -29.775) (width 0.25) (layer "F.Cu") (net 4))
 (segment (start 6.75 -9.5) (end 6.75 -5.275) (width 0.25) (layer "F.Cu") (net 4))
 (segment (start 6.75 -5.275) (end 8.275 -3.75) (width 0.25) (layer "F.Cu") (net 4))
 (segment (start 5.25 -23.775) (end 8.275 -20.75) (width 0.25) (layer "F.Cu") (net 4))
 (segment (start 14.875 -29.47335) (end 14.875 -33.358684) (width 0.25) (layer "B.Cu") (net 4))
 (segment (start 11 -23.5) (end 11.446751 -23.5) (width 0.25) (layer "B.Cu") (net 4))
 (segment (start 14.875 -33.358684) (end 10.483684 -37.75) (width 0.25) (layer "B.Cu") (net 4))
 (segment (start 10.483684 -37.75) (end 8.275 -37.75) (width 0.25) (layer "B.Cu") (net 4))
 (segment (start 11.446751 -23.5) (end 13.65 -25.703249) (width 0.25) (layer "B.Cu") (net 4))
 (segment (start 13.65 -25.703249) (end 13.65 -28.24835) (width 0.25) (layer "B.Cu") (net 4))
 (segment (start 13.65 -28.24835) (end 14.875 -29.47335) (width 0.25) (layer "B.Cu") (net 4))
 (segment (start -3.275 -37.625) (end -4.3 -36.6) (width 0.25) (layer "B.Cu") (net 3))
 (segment (start -3.275 -39.95) (end -3.275 -37.625) (width 0.25) (layer "B.Cu") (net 3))
 (segment (start -3.275 -20.625) (end -4.3 -19.6) (width 0.25) (layer "B.Cu") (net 6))
 (segment (start -3.275 -22.95) (end -3.275 -20.625) (width 0.25) (layer "B.Cu") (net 6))
 (segment (start -3.275 -3.625) (end -4.3 -2.6) (width 0.25) (layer "B.Cu") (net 8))
 (segment (start -3.275 -5.95) (end -3.275 -3.625) (width 0.25) (layer "B.Cu") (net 8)))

